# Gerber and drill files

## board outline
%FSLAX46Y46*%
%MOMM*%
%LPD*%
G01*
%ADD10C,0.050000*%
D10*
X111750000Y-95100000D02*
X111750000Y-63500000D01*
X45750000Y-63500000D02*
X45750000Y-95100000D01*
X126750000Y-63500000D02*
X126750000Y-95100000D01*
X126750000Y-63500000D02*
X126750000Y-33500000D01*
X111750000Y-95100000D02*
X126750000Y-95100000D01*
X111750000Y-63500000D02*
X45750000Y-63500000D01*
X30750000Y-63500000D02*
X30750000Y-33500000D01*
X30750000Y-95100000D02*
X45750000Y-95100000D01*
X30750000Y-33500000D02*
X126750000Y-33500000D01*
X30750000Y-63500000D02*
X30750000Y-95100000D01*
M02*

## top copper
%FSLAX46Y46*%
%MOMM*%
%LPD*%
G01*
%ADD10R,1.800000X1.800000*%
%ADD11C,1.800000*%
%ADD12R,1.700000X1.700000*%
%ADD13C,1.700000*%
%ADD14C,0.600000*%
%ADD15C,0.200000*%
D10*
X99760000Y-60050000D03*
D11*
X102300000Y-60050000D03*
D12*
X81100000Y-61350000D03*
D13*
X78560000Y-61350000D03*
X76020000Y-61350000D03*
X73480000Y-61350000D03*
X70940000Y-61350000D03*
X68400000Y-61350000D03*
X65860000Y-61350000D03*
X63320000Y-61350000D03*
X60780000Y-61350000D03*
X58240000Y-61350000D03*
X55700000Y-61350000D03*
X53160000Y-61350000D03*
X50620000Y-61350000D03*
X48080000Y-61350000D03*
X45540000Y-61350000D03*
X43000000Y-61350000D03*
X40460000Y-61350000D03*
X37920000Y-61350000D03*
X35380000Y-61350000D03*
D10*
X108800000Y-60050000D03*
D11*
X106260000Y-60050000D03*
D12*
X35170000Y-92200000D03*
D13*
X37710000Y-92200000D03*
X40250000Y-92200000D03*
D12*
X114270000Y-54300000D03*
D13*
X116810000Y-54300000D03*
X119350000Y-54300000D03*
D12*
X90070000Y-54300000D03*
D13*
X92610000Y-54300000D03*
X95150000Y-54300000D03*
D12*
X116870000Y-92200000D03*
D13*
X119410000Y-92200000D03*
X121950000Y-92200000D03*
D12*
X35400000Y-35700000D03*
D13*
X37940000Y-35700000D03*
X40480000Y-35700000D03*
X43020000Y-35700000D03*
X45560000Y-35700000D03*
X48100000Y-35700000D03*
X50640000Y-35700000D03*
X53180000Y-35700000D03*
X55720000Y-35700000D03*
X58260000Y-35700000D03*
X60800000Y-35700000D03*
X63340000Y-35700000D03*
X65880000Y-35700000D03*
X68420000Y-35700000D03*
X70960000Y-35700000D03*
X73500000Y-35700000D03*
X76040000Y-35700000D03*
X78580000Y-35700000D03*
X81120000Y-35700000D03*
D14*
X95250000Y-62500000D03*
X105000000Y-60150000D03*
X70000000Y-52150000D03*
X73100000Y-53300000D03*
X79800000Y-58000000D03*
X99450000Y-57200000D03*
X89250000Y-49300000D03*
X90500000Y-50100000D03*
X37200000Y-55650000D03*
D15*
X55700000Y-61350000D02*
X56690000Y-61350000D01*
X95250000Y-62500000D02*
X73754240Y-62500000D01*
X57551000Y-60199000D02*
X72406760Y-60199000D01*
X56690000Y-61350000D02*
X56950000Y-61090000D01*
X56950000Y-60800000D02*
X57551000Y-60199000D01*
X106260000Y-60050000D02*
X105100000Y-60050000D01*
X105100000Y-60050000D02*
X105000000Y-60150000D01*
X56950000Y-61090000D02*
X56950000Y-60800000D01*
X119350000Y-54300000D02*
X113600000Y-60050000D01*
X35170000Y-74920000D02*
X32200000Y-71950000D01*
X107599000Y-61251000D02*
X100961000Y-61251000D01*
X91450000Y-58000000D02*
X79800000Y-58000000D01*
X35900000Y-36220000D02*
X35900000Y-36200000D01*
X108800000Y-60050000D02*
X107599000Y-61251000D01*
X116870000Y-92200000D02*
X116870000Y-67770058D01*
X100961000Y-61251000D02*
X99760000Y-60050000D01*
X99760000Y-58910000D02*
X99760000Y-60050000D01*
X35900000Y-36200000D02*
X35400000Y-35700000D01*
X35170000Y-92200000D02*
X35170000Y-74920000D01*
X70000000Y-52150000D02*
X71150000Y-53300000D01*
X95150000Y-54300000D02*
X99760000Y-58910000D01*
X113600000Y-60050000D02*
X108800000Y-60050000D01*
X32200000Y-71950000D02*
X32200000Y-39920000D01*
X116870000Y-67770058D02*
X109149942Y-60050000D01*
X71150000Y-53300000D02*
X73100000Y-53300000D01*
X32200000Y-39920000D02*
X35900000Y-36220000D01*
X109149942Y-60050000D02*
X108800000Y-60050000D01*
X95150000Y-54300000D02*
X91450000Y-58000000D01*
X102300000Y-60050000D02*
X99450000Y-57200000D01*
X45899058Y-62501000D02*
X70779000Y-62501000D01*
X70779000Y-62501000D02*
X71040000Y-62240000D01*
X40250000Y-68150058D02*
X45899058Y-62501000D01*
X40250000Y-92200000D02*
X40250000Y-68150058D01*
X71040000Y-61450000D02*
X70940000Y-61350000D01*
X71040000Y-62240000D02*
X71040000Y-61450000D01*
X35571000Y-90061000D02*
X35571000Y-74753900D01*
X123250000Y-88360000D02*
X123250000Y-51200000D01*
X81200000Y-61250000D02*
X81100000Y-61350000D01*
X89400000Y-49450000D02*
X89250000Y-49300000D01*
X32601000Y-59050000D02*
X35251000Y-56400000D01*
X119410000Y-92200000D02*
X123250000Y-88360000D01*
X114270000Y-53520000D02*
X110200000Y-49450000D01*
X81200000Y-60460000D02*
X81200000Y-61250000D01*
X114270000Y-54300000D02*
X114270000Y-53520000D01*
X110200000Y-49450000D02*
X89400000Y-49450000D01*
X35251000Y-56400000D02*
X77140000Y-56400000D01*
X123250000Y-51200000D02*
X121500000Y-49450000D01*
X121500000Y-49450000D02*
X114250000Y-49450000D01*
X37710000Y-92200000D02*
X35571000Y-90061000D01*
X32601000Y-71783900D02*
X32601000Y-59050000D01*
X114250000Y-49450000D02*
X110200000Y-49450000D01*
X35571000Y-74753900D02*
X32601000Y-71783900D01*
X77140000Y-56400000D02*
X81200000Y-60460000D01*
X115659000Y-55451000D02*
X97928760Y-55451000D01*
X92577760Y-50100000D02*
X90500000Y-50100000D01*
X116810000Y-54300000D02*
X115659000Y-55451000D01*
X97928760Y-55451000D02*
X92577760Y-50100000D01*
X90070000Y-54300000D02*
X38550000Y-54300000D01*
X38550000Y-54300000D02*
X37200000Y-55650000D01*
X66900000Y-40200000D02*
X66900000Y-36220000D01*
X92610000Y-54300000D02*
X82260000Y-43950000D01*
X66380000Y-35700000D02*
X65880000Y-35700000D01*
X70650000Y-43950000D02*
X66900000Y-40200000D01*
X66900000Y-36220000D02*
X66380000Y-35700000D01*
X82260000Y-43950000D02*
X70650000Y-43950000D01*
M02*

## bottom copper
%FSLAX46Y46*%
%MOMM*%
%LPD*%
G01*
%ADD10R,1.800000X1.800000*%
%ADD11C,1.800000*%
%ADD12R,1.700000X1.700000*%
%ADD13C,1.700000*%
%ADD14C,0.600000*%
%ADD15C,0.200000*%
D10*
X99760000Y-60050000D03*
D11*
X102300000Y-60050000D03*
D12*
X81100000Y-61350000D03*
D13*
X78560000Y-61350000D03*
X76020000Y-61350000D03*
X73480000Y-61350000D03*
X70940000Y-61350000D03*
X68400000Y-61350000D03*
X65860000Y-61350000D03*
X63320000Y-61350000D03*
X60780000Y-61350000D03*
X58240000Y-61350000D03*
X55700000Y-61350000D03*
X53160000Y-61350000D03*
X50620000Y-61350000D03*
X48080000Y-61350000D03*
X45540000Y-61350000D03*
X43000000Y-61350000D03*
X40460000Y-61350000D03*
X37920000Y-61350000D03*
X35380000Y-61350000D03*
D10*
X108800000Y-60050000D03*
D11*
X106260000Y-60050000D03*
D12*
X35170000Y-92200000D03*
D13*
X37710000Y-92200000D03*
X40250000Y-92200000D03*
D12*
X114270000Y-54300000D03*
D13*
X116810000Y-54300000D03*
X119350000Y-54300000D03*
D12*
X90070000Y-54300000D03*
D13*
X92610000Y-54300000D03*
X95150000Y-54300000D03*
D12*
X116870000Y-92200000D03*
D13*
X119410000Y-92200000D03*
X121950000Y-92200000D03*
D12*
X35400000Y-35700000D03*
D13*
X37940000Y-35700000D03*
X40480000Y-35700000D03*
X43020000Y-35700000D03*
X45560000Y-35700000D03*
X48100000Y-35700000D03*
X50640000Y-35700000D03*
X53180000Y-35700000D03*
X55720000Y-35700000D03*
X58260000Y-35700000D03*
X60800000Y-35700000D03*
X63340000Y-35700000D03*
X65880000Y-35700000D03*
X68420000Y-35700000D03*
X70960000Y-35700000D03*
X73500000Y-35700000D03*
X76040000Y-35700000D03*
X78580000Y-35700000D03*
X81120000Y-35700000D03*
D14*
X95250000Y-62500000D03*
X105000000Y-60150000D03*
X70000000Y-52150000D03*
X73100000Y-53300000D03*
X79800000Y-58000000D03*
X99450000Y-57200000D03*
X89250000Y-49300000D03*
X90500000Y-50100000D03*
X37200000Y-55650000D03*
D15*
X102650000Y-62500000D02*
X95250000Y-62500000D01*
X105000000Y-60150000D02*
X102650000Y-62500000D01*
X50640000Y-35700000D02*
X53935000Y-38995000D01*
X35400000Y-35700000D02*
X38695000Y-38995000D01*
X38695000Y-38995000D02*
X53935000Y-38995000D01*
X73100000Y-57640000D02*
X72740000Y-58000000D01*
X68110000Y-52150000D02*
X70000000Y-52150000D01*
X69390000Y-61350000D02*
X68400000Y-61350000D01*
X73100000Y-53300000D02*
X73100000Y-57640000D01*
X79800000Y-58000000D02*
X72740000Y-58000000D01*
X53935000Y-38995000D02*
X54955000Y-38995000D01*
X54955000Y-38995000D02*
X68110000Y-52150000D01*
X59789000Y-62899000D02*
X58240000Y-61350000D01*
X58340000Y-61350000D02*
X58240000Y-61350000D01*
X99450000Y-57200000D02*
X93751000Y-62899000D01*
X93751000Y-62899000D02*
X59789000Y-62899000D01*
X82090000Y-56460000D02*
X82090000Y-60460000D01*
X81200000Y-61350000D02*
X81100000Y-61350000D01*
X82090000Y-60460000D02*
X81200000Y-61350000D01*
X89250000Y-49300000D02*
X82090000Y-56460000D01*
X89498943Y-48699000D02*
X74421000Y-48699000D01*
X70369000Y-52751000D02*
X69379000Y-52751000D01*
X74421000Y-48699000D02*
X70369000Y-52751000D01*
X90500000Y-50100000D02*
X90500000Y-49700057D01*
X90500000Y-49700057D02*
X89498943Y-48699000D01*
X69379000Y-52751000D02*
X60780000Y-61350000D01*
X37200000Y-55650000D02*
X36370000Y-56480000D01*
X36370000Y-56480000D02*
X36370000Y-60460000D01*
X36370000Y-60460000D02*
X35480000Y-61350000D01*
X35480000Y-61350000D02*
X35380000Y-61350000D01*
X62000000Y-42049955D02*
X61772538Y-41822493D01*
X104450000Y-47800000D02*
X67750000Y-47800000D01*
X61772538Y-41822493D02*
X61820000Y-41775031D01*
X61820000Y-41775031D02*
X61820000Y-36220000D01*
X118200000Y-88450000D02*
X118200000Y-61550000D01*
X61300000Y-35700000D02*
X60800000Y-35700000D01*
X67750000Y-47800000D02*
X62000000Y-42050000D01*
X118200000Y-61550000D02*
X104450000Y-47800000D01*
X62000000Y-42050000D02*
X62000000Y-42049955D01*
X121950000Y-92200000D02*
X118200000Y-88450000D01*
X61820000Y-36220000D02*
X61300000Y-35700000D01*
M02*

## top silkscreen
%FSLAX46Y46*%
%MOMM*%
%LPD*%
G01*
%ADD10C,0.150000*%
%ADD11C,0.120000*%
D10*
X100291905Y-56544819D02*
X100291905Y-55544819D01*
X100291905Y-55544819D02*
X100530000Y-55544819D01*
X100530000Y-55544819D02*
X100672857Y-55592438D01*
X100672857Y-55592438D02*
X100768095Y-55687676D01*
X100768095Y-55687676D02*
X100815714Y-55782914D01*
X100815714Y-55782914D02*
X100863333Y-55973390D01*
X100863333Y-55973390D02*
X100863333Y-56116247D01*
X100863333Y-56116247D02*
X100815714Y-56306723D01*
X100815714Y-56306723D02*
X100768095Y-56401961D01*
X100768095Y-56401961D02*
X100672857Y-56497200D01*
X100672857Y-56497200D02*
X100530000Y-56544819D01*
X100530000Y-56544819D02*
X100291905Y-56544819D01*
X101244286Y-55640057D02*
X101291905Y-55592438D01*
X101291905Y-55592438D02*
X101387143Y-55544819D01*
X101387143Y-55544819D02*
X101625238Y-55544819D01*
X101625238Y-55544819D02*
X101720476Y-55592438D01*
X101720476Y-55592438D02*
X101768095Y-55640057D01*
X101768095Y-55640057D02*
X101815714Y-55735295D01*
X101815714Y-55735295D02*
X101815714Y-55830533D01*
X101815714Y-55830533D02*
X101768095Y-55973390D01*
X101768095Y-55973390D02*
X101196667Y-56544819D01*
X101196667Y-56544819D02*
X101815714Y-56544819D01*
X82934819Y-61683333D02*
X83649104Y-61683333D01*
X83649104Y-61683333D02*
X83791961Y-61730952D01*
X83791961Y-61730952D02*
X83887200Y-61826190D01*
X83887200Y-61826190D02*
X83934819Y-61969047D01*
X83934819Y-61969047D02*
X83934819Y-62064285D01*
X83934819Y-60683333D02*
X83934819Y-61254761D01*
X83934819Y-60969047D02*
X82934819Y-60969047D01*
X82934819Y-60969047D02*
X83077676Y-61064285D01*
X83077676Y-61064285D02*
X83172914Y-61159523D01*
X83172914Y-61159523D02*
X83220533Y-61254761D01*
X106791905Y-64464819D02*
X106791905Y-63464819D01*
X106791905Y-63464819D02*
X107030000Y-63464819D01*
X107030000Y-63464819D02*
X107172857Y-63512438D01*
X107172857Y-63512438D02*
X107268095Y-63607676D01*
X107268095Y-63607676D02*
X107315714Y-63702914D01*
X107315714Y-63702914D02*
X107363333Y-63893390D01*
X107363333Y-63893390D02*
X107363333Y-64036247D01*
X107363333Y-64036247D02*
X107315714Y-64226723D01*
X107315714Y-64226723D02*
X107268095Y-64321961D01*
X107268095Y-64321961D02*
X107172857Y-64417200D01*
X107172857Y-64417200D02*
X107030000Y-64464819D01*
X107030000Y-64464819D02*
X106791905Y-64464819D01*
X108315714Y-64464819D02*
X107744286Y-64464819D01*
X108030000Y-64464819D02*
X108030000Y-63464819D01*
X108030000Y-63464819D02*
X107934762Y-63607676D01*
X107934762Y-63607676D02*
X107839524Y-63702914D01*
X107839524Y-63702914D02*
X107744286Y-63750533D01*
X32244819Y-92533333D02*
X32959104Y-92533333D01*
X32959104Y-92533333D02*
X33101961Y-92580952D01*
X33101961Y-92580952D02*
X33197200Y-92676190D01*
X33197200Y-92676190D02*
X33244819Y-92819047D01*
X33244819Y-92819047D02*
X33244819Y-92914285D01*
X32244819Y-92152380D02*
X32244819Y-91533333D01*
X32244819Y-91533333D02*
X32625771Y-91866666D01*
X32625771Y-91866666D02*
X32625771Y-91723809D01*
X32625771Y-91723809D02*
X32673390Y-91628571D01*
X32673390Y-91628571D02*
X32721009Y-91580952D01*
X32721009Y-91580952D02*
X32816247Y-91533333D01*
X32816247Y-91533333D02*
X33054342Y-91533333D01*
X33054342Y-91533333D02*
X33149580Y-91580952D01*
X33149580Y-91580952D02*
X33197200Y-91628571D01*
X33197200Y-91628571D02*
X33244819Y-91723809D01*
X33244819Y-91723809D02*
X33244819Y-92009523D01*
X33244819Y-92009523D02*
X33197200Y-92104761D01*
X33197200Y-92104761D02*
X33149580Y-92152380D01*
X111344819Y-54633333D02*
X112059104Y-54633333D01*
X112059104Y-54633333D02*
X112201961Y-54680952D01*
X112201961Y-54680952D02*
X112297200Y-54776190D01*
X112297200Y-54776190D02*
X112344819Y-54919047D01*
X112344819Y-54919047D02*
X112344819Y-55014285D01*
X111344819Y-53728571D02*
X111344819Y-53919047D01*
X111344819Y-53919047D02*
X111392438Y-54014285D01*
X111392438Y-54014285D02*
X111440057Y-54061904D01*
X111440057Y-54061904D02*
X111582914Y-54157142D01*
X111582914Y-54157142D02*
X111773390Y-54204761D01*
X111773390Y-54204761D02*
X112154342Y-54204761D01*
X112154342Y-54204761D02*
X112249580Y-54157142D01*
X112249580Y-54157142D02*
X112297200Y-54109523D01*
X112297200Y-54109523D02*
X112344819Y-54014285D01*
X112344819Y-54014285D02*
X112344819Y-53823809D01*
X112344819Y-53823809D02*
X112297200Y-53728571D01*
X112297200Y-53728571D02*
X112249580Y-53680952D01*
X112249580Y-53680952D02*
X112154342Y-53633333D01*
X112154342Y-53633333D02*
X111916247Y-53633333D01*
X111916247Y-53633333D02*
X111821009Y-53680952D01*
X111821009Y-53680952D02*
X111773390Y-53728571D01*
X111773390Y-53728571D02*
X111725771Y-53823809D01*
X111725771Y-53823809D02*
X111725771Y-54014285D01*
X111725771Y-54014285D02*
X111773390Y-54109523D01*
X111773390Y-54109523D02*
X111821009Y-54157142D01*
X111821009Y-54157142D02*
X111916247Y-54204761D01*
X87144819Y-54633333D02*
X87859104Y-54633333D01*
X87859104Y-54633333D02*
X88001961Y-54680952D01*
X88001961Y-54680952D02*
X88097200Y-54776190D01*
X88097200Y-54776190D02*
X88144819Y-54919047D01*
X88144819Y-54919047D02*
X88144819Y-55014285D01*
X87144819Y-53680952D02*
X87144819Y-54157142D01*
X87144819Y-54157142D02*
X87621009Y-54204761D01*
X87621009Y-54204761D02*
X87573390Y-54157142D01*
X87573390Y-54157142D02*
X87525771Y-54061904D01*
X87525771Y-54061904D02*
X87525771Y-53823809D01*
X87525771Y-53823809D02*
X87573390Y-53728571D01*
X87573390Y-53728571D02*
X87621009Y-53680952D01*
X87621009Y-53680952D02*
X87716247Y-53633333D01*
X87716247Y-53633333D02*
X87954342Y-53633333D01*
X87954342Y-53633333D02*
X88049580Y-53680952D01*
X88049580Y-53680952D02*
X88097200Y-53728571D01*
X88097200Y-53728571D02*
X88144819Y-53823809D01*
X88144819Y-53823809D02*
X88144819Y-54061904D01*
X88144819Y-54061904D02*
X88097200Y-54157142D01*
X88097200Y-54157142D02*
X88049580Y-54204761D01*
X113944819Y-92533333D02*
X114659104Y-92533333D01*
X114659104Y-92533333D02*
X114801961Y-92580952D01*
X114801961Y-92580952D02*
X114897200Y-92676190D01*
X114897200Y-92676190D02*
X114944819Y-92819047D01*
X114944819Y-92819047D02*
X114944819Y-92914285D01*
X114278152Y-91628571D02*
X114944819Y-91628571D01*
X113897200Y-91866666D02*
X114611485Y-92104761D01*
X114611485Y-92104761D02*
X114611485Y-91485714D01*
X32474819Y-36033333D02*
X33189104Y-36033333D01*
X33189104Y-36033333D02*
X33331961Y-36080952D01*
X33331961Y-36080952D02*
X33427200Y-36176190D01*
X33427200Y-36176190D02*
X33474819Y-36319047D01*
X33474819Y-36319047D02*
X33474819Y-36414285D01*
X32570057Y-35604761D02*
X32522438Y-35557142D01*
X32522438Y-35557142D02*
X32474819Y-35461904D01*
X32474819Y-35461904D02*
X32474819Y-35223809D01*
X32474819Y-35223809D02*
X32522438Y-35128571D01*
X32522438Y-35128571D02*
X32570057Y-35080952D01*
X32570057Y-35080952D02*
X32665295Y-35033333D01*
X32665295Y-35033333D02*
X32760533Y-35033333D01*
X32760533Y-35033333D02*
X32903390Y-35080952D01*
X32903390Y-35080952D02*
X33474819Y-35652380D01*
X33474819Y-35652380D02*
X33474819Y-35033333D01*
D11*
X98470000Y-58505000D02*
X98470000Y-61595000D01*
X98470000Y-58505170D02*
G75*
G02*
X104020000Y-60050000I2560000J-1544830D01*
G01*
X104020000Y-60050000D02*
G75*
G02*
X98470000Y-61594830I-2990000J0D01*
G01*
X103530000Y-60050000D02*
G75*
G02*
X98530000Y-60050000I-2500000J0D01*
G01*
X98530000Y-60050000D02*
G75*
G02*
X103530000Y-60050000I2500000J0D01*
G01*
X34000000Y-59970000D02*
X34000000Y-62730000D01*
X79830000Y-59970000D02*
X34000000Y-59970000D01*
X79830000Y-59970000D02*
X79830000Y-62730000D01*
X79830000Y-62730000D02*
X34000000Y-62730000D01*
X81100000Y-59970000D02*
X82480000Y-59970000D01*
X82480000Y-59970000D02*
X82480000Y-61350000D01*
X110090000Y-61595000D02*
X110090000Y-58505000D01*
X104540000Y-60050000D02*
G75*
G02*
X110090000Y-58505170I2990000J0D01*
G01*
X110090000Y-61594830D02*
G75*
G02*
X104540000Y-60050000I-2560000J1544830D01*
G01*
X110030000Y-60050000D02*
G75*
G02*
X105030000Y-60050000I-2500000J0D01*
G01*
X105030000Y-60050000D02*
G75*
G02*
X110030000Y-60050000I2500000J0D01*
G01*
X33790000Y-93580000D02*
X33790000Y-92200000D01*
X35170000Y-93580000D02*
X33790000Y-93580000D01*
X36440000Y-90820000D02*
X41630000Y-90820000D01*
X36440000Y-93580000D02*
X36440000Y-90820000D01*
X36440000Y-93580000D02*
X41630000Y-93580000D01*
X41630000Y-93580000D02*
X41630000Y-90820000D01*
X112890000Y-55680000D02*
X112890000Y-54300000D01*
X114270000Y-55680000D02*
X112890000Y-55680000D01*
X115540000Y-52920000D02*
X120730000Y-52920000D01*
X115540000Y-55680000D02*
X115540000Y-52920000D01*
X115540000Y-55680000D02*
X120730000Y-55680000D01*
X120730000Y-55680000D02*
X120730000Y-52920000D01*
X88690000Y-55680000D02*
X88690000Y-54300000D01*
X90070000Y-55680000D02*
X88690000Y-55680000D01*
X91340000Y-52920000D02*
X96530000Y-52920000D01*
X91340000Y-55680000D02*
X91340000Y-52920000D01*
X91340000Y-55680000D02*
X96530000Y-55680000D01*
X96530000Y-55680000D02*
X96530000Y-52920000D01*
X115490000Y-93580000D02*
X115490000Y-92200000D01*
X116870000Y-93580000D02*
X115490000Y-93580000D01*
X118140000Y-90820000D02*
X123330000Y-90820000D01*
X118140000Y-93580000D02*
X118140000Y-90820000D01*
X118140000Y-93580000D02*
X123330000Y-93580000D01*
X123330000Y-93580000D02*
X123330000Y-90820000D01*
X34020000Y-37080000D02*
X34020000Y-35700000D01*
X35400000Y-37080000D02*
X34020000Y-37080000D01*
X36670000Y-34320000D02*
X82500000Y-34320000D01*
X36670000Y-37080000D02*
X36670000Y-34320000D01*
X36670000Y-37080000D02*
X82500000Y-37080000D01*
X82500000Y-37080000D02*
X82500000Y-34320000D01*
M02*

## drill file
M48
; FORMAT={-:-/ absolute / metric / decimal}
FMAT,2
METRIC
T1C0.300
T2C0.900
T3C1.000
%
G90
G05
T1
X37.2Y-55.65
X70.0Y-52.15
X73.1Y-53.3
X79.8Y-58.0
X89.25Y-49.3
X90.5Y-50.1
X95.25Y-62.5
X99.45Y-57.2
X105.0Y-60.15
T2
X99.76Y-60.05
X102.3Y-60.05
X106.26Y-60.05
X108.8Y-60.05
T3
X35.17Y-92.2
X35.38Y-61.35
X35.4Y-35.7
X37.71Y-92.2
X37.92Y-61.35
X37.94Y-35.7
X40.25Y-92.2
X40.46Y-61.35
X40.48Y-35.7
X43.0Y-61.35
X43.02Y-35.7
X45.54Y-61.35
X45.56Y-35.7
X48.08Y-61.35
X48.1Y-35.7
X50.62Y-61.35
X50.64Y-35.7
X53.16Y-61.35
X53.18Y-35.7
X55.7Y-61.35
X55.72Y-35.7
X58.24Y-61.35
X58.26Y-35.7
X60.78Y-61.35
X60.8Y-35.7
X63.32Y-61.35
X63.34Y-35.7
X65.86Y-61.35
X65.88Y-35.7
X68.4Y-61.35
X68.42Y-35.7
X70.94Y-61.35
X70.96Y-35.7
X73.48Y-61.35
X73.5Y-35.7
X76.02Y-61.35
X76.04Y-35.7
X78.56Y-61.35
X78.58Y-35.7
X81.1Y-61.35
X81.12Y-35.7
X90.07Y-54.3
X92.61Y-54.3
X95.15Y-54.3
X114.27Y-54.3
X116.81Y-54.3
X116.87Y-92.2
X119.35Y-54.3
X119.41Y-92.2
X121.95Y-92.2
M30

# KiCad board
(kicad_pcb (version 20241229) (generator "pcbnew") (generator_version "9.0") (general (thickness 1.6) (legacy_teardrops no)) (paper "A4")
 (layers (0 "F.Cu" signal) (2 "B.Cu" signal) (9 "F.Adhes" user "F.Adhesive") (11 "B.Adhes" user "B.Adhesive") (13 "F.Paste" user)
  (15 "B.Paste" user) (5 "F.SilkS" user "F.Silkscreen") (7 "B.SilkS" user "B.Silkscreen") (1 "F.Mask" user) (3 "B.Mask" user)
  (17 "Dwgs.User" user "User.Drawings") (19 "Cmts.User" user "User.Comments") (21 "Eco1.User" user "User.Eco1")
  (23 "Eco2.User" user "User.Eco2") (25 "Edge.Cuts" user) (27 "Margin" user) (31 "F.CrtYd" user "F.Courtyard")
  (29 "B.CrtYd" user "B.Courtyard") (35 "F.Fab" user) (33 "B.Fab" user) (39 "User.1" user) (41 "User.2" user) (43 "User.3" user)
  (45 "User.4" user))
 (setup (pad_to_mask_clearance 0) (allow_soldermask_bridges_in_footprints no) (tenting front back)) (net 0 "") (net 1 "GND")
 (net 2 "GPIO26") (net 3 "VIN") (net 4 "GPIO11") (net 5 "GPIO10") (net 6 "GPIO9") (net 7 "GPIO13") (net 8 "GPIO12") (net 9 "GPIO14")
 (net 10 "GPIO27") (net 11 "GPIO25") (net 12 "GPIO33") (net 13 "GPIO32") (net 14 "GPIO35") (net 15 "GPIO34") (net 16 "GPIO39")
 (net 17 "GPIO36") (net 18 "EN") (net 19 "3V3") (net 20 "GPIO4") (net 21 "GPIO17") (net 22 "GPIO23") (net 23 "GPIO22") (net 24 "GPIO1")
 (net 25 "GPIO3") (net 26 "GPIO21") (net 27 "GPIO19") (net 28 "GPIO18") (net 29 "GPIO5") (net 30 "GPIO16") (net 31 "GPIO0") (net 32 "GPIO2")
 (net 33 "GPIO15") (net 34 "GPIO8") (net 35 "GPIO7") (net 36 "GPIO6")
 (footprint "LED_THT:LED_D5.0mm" (layer "F.Cu") (at 99.76 60.05)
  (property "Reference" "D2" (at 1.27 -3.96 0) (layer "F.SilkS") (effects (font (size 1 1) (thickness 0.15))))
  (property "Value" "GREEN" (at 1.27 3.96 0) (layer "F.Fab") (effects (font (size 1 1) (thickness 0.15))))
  (fp_line (start -1.29 -1.545) (end -1.29 1.545) (stroke (width 0.12) (type solid)) (layer "F.SilkS"))
  (fp_arc (start -1.29 -1.54483) (mid 2.071779 -2.880495) (end 4.26 0) (stroke (width 0.12) (type solid)) (layer "F.SilkS"))
  (fp_arc (start 4.26 0) (mid 2.071779 2.880495) (end -1.29 1.54483) (stroke (width 0.12) (type solid)) (layer "F.SilkS"))
  (fp_circle (center 1.27 0) (end 3.77 0) (stroke (width 0.12) (type solid)) (fill no) (layer "F.SilkS"))
  (pad "1" thru_hole rect (at 0 0) (size 1.8 1.8) (drill 0.9) (layers "*.Cu" "*.Mask") (remove_unused_layers no) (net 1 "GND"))
  (pad "2" thru_hole circle (at 2.54 0) (size 1.8 1.8) (drill 0.9) (layers "*.Cu" "*.Mask") (remove_unused_layers no) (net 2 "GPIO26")))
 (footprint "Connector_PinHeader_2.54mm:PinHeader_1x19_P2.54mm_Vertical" (layer "F.Cu") (at 81.1 61.35 -90)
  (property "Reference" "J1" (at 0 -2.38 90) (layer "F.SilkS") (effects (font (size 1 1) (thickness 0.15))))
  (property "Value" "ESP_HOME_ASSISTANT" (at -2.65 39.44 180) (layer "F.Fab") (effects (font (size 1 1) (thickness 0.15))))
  (fp_line (start -1.38 47.1) (end 1.38 47.1) (stroke (width 0.12) (type solid)) (layer "F.SilkS"))
  (fp_line (start -1.38 1.27) (end -1.38 47.1) (stroke (width 0.12) (type solid)) (layer "F.SilkS"))
  (fp_line (start -1.38 1.27) (end 1.38 1.27) (stroke (width 0.12) (type solid)) (layer "F.SilkS"))
  (fp_line (start 1.38 1.27) (end 1.38 47.1) (stroke (width 0.12) (type solid)) (layer "F.SilkS"))
  (fp_line (start -1.38 0) (end -1.38 -1.38) (stroke (width 0.12) (type solid)) (layer "F.SilkS"))
  (fp_line (start -1.38 -1.38) (end 0 -1.38) (stroke (width 0.12) (type solid)) (layer "F.SilkS"))
  (pad "1" thru_hole rect (at 0 0 270) (size 1.7 1.7) (drill 1) (layers "*.Cu" "*.Mask") (remove_unused_layers no) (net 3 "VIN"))
  (pad "2" thru_hole circle (at 0 2.54 270) (size 1.7 1.7) (drill 1) (layers "*.Cu" "*.Mask") (remove_unused_layers no) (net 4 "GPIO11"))
  (pad "3" thru_hole circle (at 0 5.08 270) (size 1.7 1.7) (drill 1) (layers "*.Cu" "*.Mask") (remove_unused_layers no) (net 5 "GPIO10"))
  (pad "4" thru_hole circle (at 0 7.62 270) (size 1.7 1.7) (drill 1) (layers "*.Cu" "*.Mask") (remove_unused_layers no) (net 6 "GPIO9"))
  (pad "5" thru_hole circle (at 0 10.16 270) (size 1.7 1.7) (drill 1) (layers "*.Cu" "*.Mask") (remove_unused_layers no) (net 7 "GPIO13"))
  (pad "6" thru_hole circle (at 0 12.7 270) (size 1.7 1.7) (drill 1) (layers "*.Cu" "*.Mask") (remove_unused_layers no) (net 1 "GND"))
  (pad "7" thru_hole circle (at 0 15.24 270) (size 1.7 1.7) (drill 1) (layers "*.Cu" "*.Mask") (remove_unused_layers no) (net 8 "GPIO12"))
  (pad "8" thru_hole circle (at 0 17.78 270) (size 1.7 1.7) (drill 1) (layers "*.Cu" "*.Mask") (remove_unused_layers no) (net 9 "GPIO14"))
  (pad "9" thru_hole circle (at 0 20.32 270) (size 1.7 1.7) (drill 1) (layers "*.Cu" "*.Mask") (remove_unused_layers no) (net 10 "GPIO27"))
  (pad "10" thru_hole circle (at 0 22.86 270) (size 1.7 1.7) (drill 1) (layers "*.Cu" "*.Mask") (remove_unused_layers no) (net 2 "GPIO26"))
  (pad "11" thru_hole circle (at 0 25.4 270) (size 1.7 1.7) (drill 1) (layers "*.Cu" "*.Mask") (remove_unused_layers no) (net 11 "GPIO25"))
  (pad "12" thru_hole circle (at 0 27.94 270) (size 1.7 1.7) (drill 1) (layers "*.Cu" "*.Mask") (remove_unused_layers no) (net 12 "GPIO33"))
  (pad "13" thru_hole circle (at 0 30.48 270) (size 1.7 1.7) (drill 1) (layers "*.Cu" "*.Mask") (remove_unused_layers no) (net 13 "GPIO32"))
  (pad "14" thru_hole circle (at 0 33.02 270) (size 1.7 1.7) (drill 1) (layers "*.Cu" "*.Mask") (remove_unused_layers no) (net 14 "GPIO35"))
  (pad "15" thru_hole circle (at 0 35.56 270) (size 1.7 1.7) (drill 1) (layers "*.Cu" "*.Mask") (remove_unused_layers no) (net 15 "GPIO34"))
  (pad "16" thru_hole circle (at 0 38.1 270) (size 1.7 1.7) (drill 1) (layers "*.Cu" "*.Mask") (remove_unused_layers no) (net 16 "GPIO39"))
  (pad "17" thru_hole circle (at 0 40.64 270) (size 1.7 1.7) (drill 1) (layers "*.Cu" "*.Mask") (remove_unused_layers no) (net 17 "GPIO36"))
  (pad "18" thru_hole circle (at 0 43.18 270) (size 1.7 1.7) (drill 1) (layers "*.Cu" "*.Mask") (remove_unused_layers no) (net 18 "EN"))
  (pad "19" thru_hole circle (at 0 45.72 270) (size 1.7 1.7) (drill 1) (layers "*.Cu" "*.Mask") (remove_unused_layers no) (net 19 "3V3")))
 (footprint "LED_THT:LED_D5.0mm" (layer "F.Cu") (at 108.8 60.05 180)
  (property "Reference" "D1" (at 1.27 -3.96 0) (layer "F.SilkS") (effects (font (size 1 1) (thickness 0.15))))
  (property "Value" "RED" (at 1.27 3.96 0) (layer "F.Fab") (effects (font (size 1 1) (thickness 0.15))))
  (fp_line (start -1.29 -1.545) (end -1.29 1.545) (stroke (width 0.12) (type solid)) (layer "F.SilkS"))
  (fp_arc (start 4.26 0) (mid 2.071779 2.880495) (end -1.29 1.54483) (stroke (width 0.12) (type solid)) (layer "F.SilkS"))
  (fp_arc (start -1.29 -1.54483) (mid 2.071779 -2.880495) (end 4.26 0) (stroke (width 0.12) (type solid)) (layer "F.SilkS"))
  (fp_circle (center 1.27 0) (end 3.77 0) (stroke (width 0.12) (type solid)) (fill no) (layer "F.SilkS"))
  (pad "1" thru_hole rect (at 0 0 180) (size 1.8 1.8) (drill 0.9) (layers "*.Cu" "*.Mask") (remove_unused_layers no) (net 1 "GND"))
  (pad "2" thru_hole circle (at 2.54 0 180) (size 1.8 1.8) (drill 0.9) (layers "*.Cu" "*.Mask") (remove_unused_layers no) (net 11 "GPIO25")))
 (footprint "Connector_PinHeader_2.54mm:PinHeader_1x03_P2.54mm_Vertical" (layer "F.Cu") (at 35.17 92.2 90)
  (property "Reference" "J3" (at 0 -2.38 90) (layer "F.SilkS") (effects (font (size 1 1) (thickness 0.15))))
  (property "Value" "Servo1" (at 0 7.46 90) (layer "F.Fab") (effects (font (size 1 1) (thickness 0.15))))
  (fp_line (start -1.38 -1.38) (end 0 -1.38) (stroke (width 0.12) (type solid)) (layer "F.SilkS"))
  (fp_line (start -1.38 0) (end -1.38 -1.38) (stroke (width 0.12) (type solid)) (layer "F.SilkS"))
  (fp_line (start 1.38 1.27) (end 1.38 6.46) (stroke (width 0.12) (type solid)) (layer "F.SilkS"))
  (fp_line (start -1.38 1.27) (end 1.38 1.27) (stroke (width 0.12) (type solid)) (layer "F.SilkS"))
  (fp_line (start -1.38 1.27) (end -1.38 6.46) (stroke (width 0.12) (type solid)) (layer "F.SilkS"))
  (fp_line (start -1.38 6.46) (end 1.38 6.46) (stroke (width 0.12) (type solid)) (layer "F.SilkS"))
  (pad "1" thru_hole rect (at 0 0 90) (size 1.7 1.7) (drill 1) (layers "*.Cu" "*.Mask") (remove_unused_layers no) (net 1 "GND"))
  (pad "2" thru_hole circle (at 0 2.54 90) (size 1.7 1.7) (drill 1) (layers "*.Cu" "*.Mask") (remove_unused_layers no) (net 3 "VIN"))
  (pad "3" thru_hole circle (at 0 5.08 90) (size 1.7 1.7) (drill 1) (layers "*.Cu" "*.Mask") (remove_unused_layers no) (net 7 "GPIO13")))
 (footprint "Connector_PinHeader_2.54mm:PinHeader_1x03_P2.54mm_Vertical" (layer "F.Cu") (at 114.27 54.3 90)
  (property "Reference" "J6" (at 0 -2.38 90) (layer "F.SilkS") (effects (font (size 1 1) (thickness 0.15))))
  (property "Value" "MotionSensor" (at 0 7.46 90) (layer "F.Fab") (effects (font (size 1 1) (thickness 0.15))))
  (fp_line (start -1.38 -1.38) (end 0 -1.38) (stroke (width 0.12) (type solid)) (layer "F.SilkS"))
  (fp_line (start -1.38 0) (end -1.38 -1.38) (stroke (width 0.12) (type solid)) (layer "F.SilkS"))
  (fp_line (start 1.38 1.27) (end 1.38 6.46) (stroke (width 0.12) (type solid)) (layer "F.SilkS"))
  (fp_line (start -1.38 1.27) (end 1.38 1.27) (stroke (width 0.12) (type solid)) (layer "F.SilkS"))
  (fp_line (start -1.38 1.27) (end -1.38 6.46) (stroke (width 0.12) (type solid)) (layer "F.SilkS"))
  (fp_line (start -1.38 6.46) (end 1.38 6.46) (stroke (width 0.12) (type solid)) (layer "F.SilkS"))
  (pad "1" thru_hole rect (at 0 0 90) (size 1.7 1.7) (drill 1) (layers "*.Cu" "*.Mask") (remove_unused_layers no) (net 3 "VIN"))
  (pad "2" thru_hole circle (at 0 2.54 90) (size 1.7 1.7) (drill 1) (layers "*.Cu" "*.Mask") (remove_unused_layers no) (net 10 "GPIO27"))
  (pad "3" thru_hole circle (at 0 5.08 90) (size 1.7 1.7) (drill 1) (layers "*.Cu" "*.Mask") (remove_unused_layers no) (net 1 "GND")))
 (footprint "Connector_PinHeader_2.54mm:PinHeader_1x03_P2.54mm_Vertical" (layer "F.Cu") (at 90.07 54.3 90)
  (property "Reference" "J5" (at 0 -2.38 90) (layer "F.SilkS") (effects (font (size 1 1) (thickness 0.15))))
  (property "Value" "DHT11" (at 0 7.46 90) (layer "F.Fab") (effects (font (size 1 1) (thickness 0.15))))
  (fp_line (start -1.38 -1.38) (end 0 -1.38) (stroke (width 0.12) (type solid)) (layer "F.SilkS"))
  (fp_line (start -1.38 0) (end -1.38 -1.38) (stroke (width 0.12) (type solid)) (layer "F.SilkS"))
  (fp_line (start 1.38 1.27) (end 1.38 6.46) (stroke (width 0.12) (type solid)) (layer "F.SilkS"))
  (fp_line (start -1.38 1.27) (end 1.38 1.27) (stroke (width 0.12) (type solid)) (layer "F.SilkS"))
  (fp_line (start -1.38 1.27) (end -1.38 6.46) (stroke (width 0.12) (type solid)) (layer "F.SilkS"))
  (fp_line (start -1.38 6.46) (end 1.38 6.46) (stroke (width 0.12) (type solid)) (layer "F.SilkS"))
  (pad "1" thru_hole rect (at 0 0 90) (size 1.7 1.7) (drill 1) (layers "*.Cu" "*.Mask") (remove_unused_layers no) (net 19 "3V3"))
  (pad "2" thru_hole circle (at 0 2.54 90) (size 1.7 1.7) (drill 1) (layers "*.Cu" "*.Mask") (remove_unused_layers no) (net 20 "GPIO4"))
  (pad "3" thru_hole circle (at 0 5.08 90) (size 1.7 1.7) (drill 1) (layers "*.Cu" "*.Mask") (remove_unused_layers no) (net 1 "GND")))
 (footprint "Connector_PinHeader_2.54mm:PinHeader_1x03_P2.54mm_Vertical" (layer "F.Cu") (at 116.87 92.2 90)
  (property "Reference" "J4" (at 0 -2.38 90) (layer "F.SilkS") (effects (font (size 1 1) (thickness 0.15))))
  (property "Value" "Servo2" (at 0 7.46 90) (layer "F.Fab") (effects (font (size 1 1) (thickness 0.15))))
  (fp_line (start -1.38 -1.38) (end 0 -1.38) (stroke (width 0.12) (type solid)) (layer "F.SilkS"))
  (fp_line (start -1.38 0) (end -1.38 -1.38) (stroke (width 0.12) (type solid)) (layer "F.SilkS"))
  (fp_line (start 1.38 1.27) (end 1.38 6.46) (stroke (width 0.12) (type solid)) (layer "F.SilkS"))
  (fp_line (start -1.38 1.27) (end 1.38 1.27) (stroke (width 0.12) (type solid)) (layer "F.SilkS"))
  (fp_line (start -1.38 1.27) (end -1.38 6.46) (stroke (width 0.12) (type solid)) (layer "F.SilkS"))
  (fp_line (start -1.38 6.46) (end 1.38 6.46) (stroke (width 0.12) (type solid)) (layer "F.SilkS"))
  (pad "1" thru_hole rect (at 0 0 90) (size 1.7 1.7) (drill 1) (layers "*.Cu" "*.Mask") (remove_unused_layers no) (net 1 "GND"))
  (pad "2" thru_hole circle (at 0 2.54 90) (size 1.7 1.7) (drill 1) (layers "*.Cu" "*.Mask") (remove_unused_layers no) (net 3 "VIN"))
  (pad "3" thru_hole circle (at 0 5.08 90) (size 1.7 1.7) (drill 1) (layers "*.Cu" "*.Mask") (remove_unused_layers no) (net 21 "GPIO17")))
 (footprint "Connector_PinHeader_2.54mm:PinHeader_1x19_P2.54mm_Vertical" (layer "F.Cu") (at 35.4 35.7 90)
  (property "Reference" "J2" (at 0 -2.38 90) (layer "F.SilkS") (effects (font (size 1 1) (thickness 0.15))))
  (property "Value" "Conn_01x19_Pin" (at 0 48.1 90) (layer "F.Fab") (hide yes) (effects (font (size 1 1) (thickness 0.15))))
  (fp_line (start -1.38 -1.38) (end 0 -1.38) (stroke (width 0.12) (type solid)) (layer "F.SilkS"))
  (fp_line (start -1.38 0) (end -1.38 -1.38) (stroke (width 0.12) (type solid)) (layer "F.SilkS"))
  (fp_line (start 1.38 1.27) (end 1.38 47.1) (stroke (width 0.12) (type solid)) (layer "F.SilkS"))
  (fp_line (start -1.38 1.27) (end 1.38 1.27) (stroke (width 0.12) (type solid)) (layer "F.SilkS"))
  (fp_line (start -1.38 1.27) (end -1.38 47.1) (stroke (width 0.12) (type solid)) (layer "F.SilkS"))
  (fp_line (start -1.38 47.1) (end 1.38 47.1) (stroke (width 0.12) (type solid)) (layer "F.SilkS"))
  (pad "1" thru_hole rect (at 0 0 90) (size 1.7 1.7) (drill 1) (layers "*.Cu" "*.Mask") (remove_unused_layers no) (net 1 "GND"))
  (pad "2" thru_hole circle (at 0 2.54 90) (size 1.7 1.7) (drill 1) (layers "*.Cu" "*.Mask") (remove_unused_layers no) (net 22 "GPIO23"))
  (pad "3" thru_hole circle (at 0 5.08 90) (size 1.7 1.7) (drill 1) (layers "*.Cu" "*.Mask") (remove_unused_layers no) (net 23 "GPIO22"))
  (pad "4" thru_hole circle (at 0 7.62 90) (size 1.7 1.7) (drill 1) (layers "*.Cu" "*.Mask") (remove_unused_layers no) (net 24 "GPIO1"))
  (pad "5" thru_hole circle (at 0 10.16 90) (size 1.7 1.7) (drill 1) (layers "*.Cu" "*.Mask") (remove_unused_layers no) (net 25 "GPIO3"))
  (pad "6" thru_hole circle (at 0 12.7 90) (size 1.7 1.7) (drill 1) (layers "*.Cu" "*.Mask") (remove_unused_layers no) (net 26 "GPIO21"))
  (pad "7" thru_hole circle (at 0 15.24 90) (size 1.7 1.7) (drill 1) (layers "*.Cu" "*.Mask") (remove_unused_layers no) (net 1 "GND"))
  (pad "8" thru_hole circle (at 0 17.78 90) (size 1.7 1.7) (drill 1) (layers "*.Cu" "*.Mask") (remove_unused_layers no) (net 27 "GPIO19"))
  (pad "9" thru_hole circle (at 0 20.32 90) (size 1.7 1.7) (drill 1) (layers "*.Cu" "*.Mask") (remove_unused_layers no) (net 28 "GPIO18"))
  (pad "10" thru_hole circle (at 0 22.86 90) (size 1.7 1.7) (drill 1) (layers "*.Cu" "*.Mask") (remove_unused_layers no) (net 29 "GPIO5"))
  (pad "11" thru_hole circle (at 0 25.4 90) (size 1.7 1.7) (drill 1) (layers "*.Cu" "*.Mask") (remove_unused_layers no) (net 21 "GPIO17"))
  (pad "12" thru_hole circle (at 0 27.94 90) (size 1.7 1.7) (drill 1) (layers "*.Cu" "*.Mask") (remove_unused_layers no) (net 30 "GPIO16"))
  (pad "13" thru_hole circle (at 0 30.48 90) (size 1.7 1.7) (drill 1) (layers "*.Cu" "*.Mask") (remove_unused_layers no) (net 20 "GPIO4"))
  (pad "14" thru_hole circle (at 0 33.02 90) (size 1.7 1.7) (drill 1) (layers "*.Cu" "*.Mask") (remove_unused_layers no) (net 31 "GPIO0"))
  (pad "15" thru_hole circle (at 0 35.56 90) (size 1.7 1.7) (drill 1) (layers "*.Cu" "*.Mask") (remove_unused_layers no) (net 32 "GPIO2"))
  (pad "16" thru_hole circle (at 0 38.1 90) (size 1.7 1.7) (drill 1) (layers "*.Cu" "*.Mask") (remove_unused_layers no) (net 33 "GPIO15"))
  (pad "17" thru_hole circle (at 0 40.64 90) (size 1.7 1.7) (drill 1) (layers "*.Cu" "*.Mask") (remove_unused_layers no) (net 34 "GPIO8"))
  (pad "18" thru_hole circle (at 0 43.18 90) (size 1.7 1.7) (drill 1) (layers "*.Cu" "*.Mask") (remove_unused_layers no) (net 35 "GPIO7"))
  (pad "19" thru_hole circle (at 0 45.72 90) (size 1.7 1.7) (drill 1) (layers "*.Cu" "*.Mask") (remove_unused_layers no) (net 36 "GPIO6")))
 (gr_line (start 111.75 95.1) (end 111.75 63.5) (stroke (width 0.05) (type default)) (layer "Edge.Cuts"))
 (gr_line (start 45.75 63.5) (end 45.75 95.1) (stroke (width 0.05) (type default)) (layer "Edge.Cuts"))
 (gr_line (start 126.75 63.5) (end 126.75 95.1) (stroke (width 0.05) (type default)) (layer "Edge.Cuts"))
 (gr_line (start 126.75 63.5) (end 126.75 33.5) (stroke (width 0.05) (type default)) (layer "Edge.Cuts"))
 (gr_line (start 111.75 95.1) (end 126.75 95.1) (stroke (width 0.05) (type default)) (layer "Edge.Cuts"))
 (gr_line (start 111.75 63.5) (end 45.75 63.5) (stroke (width 0.05) (type default)) (layer "Edge.Cuts"))
 (gr_line (start 30.75 63.5) (end 30.75 33.5) (stroke (width 0.05) (type default)) (layer "Edge.Cuts"))
 (gr_line (start 30.75 95.1) (end 45.75 95.1) (stroke (width 0.05) (type default)) (layer "Edge.Cuts"))
 (gr_line (start 30.75 33.5) (end 126.75 33.5) (stroke (width 0.05) (type default)) (layer "Edge.Cuts"))
 (gr_line (start 30.75 63.5) (end 30.75 95.1) (stroke (width 0.05) (type default)) (layer "Edge.Cuts"))
 (segment (start 55.7 61.35) (end 56.69 61.35) (width 0.2) (layer "F.Cu") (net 11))
 (segment (start 95.25 62.5) (end 73.75424 62.5) (width 0.2) (layer "F.Cu") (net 11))
 (segment (start 57.551 60.199) (end 72.40676 60.199) (width 0.2) (layer "F.Cu") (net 11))
 (segment (start 56.69 61.35) (end 56.95 61.09) (width 0.2) (layer "F.Cu") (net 11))
 (segment (start 56.95 60.8) (end 57.551 60.199) (width 0.2) (layer "F.Cu") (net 11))
 (segment (start 106.26 60.05) (end 105.1 60.05) (width 0.2) (layer "F.Cu") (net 11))
 (segment (start 105.1 60.05) (end 105 60.15) (width 0.2) (layer "F.Cu") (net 11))
 (segment (start 56.95 61.09) (end 56.95 60.8) (width 0.2) (layer "F.Cu") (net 11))
 (via (at 95.25 62.5) (size 0.6) (drill 0.3) (layers "F.Cu" "B.Cu") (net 11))
 (via (at 105 60.15) (size 0.6) (drill 0.3) (layers "F.Cu" "B.Cu") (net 11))
 (segment (start 102.65 62.5) (end 95.25 62.5) (width 0.2) (layer "B.Cu") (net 11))
 (segment (start 105 60.15) (end 102.65 62.5) (width 0.2) (layer "B.Cu") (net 11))
 (segment (start 119.35 54.3) (end 113.6 60.05) (width 0.2) (layer "F.Cu") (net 1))
 (segment (start 35.17 74.92) (end 32.2 71.95) (width 0.2) (layer "F.Cu") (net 1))
 (segment (start 107.599 61.251) (end 100.961 61.251) (width 0.2) (layer "F.Cu") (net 1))
 (segment (start 91.45 58) (end 79.8 58) (width 0.2) (layer "F.Cu") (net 1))
 (segment (start 35.9 36.22) (end 35.9 36.2) (width 0.2) (layer "F.Cu") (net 1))
 (segment (start 108.8 60.05) (end 107.599 61.251) (width 0.2) (layer "F.Cu") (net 1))
 (segment (start 116.87 92.2) (end 116.87 67.770058) (width 0.2) (layer "F.Cu") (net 1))
 (segment (start 100.961 61.251) (end 99.76 60.05) (width 0.2) (layer "F.Cu") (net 1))
 (segment (start 99.76 58.91) (end 99.76 60.05) (width 0.2) (layer "F.Cu") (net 1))
 (segment (start 35.9 36.2) (end 35.4 35.7) (width 0.2) (layer "F.Cu") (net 1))
 (segment (start 35.17 92.2) (end 35.17 74.92) (width 0.2) (layer "F.Cu") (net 1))
 (segment (start 70 52.15) (end 71.15 53.3) (width 0.2) (layer "F.Cu") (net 1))
 (segment (start 95.15 54.3) (end 99.76 58.91) (width 0.2) (layer "F.Cu") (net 1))
 (segment (start 113.6 60.05) (end 108.8 60.05) (width 0.2) (layer "F.Cu") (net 1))
 (segment (start 32.2 71.95) (end 32.2 39.92) (width 0.2) (layer "F.Cu") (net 1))
 (segment (start 116.87 67.770058) (end 109.149942 60.05) (width 0.2) (layer "F.Cu") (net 1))
 (segment (start 71.15 53.3) (end 73.1 53.3) (width 0.2) (layer "F.Cu") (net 1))
 (segment (start 32.2 39.92) (end 35.9 36.22) (width 0.2) (layer "F.Cu") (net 1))
 (segment (start 109.149942 60.05) (end 108.8 60.05) (width 0.2) (layer "F.Cu") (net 1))
 (segment (start 95.15 54.3) (end 91.45 58) (width 0.2) (layer "F.Cu") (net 1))
 (via (at 70 52.15) (size 0.6) (drill 0.3) (layers "F.Cu" "B.Cu") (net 1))
 (via (at 73.1 53.3) (size 0.6) (drill 0.3) (layers "F.Cu" "B.Cu") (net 1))
 (via (at 79.8 58) (size 0.6) (drill 0.3) (layers "F.Cu" "B.Cu") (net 1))
 (segment (start 50.64 35.7) (end 53.935 38.995) (width 0.2) (layer "B.Cu") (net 1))
 (segment (start 35.4 35.7) (end 38.695 38.995) (width 0.2) (layer "B.Cu") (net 1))
 (segment (start 38.695 38.995) (end 53.935 38.995) (width 0.2) (layer "B.Cu") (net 1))
 (segment (start 73.1 57.64) (end 72.74 58) (width 0.2) (layer "B.Cu") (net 1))
 (segment (start 68.11 52.15) (end 70 52.15) (width 0.2) (layer "B.Cu") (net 1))
 (segment (start 69.39 61.35) (end 68.4 61.35) (width 0.2) (layer "B.Cu") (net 1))
 (segment (start 73.1 53.3) (end 73.1 57.64) (width 0.2) (layer "B.Cu") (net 1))
 (segment (start 79.8 58) (end 72.74 58) (width 0.2) (layer "B.Cu") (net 1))
 (segment (start 53.935 38.995) (end 54.955 38.995) (width 0.2) (layer "B.Cu") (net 1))
 (segment (start 54.955 38.995) (end 68.11 52.15) (width 0.2) (layer "B.Cu") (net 1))
 (segment (start 102.3 60.05) (end 99.45 57.2) (width 0.2) (layer "F.Cu") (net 2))
 (via (at 99.45 57.2) (size 0.6) (drill 0.3) (layers "F.Cu" "B.Cu") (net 2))
 (segment (start 59.789 62.899) (end 58.24 61.35) (width 0.2) (layer "B.Cu") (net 2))
 (segment (start 58.34 61.35) (end 58.24 61.35) (width 0.2) (layer "B.Cu") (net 2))
 (segment (start 99.45 57.2) (end 93.751 62.899) (width 0.2) (layer "B.Cu") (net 2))
 (segment (start 93.751 62.899) (end 59.789 62.899) (width 0.2) (layer "B.Cu") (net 2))
 (segment (start 45.899058 62.501) (end 70.779 62.501) (width 0.2) (layer "F.Cu") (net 7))
 (segment (start 70.779 62.501) (end 71.04 62.24) (width 0.2) (layer "F.Cu") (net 7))
 (segment (start 40.25 68.150058) (end 45.899058 62.501) (width 0.2) (layer "F.Cu") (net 7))
 (segment (start 40.25 92.2) (end 40.25 68.150058) (width 0.2) (layer "F.Cu") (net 7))
 (segment (start 71.04 61.45) (end 70.94 61.35) (width 0.2) (layer "F.Cu") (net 7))
 (segment (start 71.04 62.24) (end 71.04 61.45) (width 0.2) (layer "F.Cu") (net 7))
 (segment (start 35.571 90.061) (end 35.571 74.7539) (width 0.2) (layer "F.Cu") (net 3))
 (segment (start 123.25 88.36) (end 123.25 51.2) (width 0.2) (layer "F.Cu") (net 3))
 (segment (start 81.2 61.25) (end 81.1 61.35) (width 0.2) (layer "F.Cu") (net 3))
 (segment (start 89.4 49.45) (end 89.25 49.3) (width 0.2) (layer "F.Cu") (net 3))
 (segment (start 32.601 59.05) (end 35.251 56.4) (width 0.2) (layer "F.Cu") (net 3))
 (segment (start 119.41 92.2) (end 123.25 88.36) (width 0.2) (layer "F.Cu") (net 3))
 (segment (start 114.27 53.52) (end 110.2 49.45) (width 0.2) (layer "F.Cu") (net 3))
 (segment (start 81.2 60.46) (end 81.2 61.25) (width 0.2) (layer "F.Cu") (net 3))
 (segment (start 114.27 54.3) (end 114.27 53.52) (width 0.2) (layer "F.Cu") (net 3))
 (segment (start 110.2 49.45) (end 89.4 49.45) (width 0.2) (layer "F.Cu") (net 3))
 (segment (start 35.251 56.4) (end 77.14 56.4) (width 0.2) (layer "F.Cu") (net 3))
 (segment (start 123.25 51.2) (end 121.5 49.45) (width 0.2) (layer "F.Cu") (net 3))
 (segment (start 121.5 49.45) (end 114.25 49.45) (width 0.2) (layer "F.Cu") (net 3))
 (segment (start 37.71 92.2) (end 35.571 90.061) (width 0.2) (layer "F.Cu") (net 3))
 (segment (start 32.601 71.7839) (end 32.601 59.05) (width 0.2) (layer "F.Cu") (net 3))
 (segment (start 114.25 49.45) (end 110.2 49.45) (width 0.2) (layer "F.Cu") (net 3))
 (segment (start 35.571 74.7539) (end 32.601 71.7839) (width 0.2) (layer "F.Cu") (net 3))
 (segment (start 77.14 56.4) (end 81.2 60.46) (width 0.2) (layer "F.Cu") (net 3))
 (via (at 89.25 49.3) (size 0.6) (drill 0.3) (layers "F.Cu" "B.Cu") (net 3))
 (segment (start 82.09 56.46) (end 82.09 60.46) (width 0.2) (layer "B.Cu") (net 3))
 (segment (start 81.2 61.35) (end 81.1 61.35) (width 0.2) (layer "B.Cu") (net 3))
 (segment (start 82.09 60.46) (end 81.2 61.35) (width 0.2) (layer "B.Cu") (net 3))
 (segment (start 89.25 49.3) (end 82.09 56.46) (width 0.2) (layer "B.Cu") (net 3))
 (segment (start 115.659 55.451) (end 97.92876 55.451) (width 0.2) (layer "F.Cu") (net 10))
 (segment (start 92.57776 50.1) (end 90.5 50.1) (width 0.2) (layer "F.Cu") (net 10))
 (segment (start 116.81 54.3) (end 115.659 55.451) (width 0.2) (layer "F.Cu") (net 10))
 (segment (start 97.92876 55.451) (end 92.57776 50.1) (width 0.2) (layer "F.Cu") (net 10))
 (via (at 90.5 50.1) (size 0.6) (drill 0.3) (layers "F.Cu" "B.Cu") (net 10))
 (segment (start 89.498943 48.699) (end 74.421 48.699) (width 0.2) (layer "B.Cu") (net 10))
 (segment (start 70.369 52.751) (end 69.379 52.751) (width 0.2) (layer "B.Cu") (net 10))
 (segment (start 74.421 48.699) (end 70.369 52.751) (width 0.2) (layer "B.Cu") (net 10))
 (segment (start 90.5 50.1) (end 90.5 49.700057) (width 0.2) (layer "B.Cu") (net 10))
 (segment (start 90.5 49.700057) (end 89.498943 48.699) (width 0.2) (layer "B.Cu") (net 10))
 (segment (start 69.379 52.751) (end 60.78 61.35) (width 0.2) (layer "B.Cu") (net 10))
 (segment (start 90.07 54.3) (end 38.55 54.3) (width 0.2) (layer "F.Cu") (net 19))
 (segment (start 38.55 54.3) (end 37.2 55.65) (width 0.2) (layer "F.Cu") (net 19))
 (via (at 37.2 55.65) (size 0.6) (drill 0.3) (layers "F.Cu" "B.Cu") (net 19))
 (segment (start 37.2 55.65) (end 36.37 56.48) (width 0.2) (layer "B.Cu") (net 19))
 (segment (start 36.37 56.48) (end 36.37 60.46) (width 0.2) (layer "B.Cu") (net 19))
 (segment (start 36.37 60.46) (end 35.48 61.35) (width 0.2) (layer "B.Cu") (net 19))
 (segment (start 35.48 61.35) (end 35.38 61.35) (width 0.2) (layer "B.Cu") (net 19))
 (segment (start 66.9 40.2) (end 66.9 36.22) (width 0.2) (layer "F.Cu") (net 20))
 (segment (start 92.61 54.3) (end 82.26 43.95) (width 0.2) (layer "F.Cu") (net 20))
 (segment (start 66.38 35.7) (end 65.88 35.7) (width 0.2) (layer "F.Cu") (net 20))
 (segment (start 70.65 43.95) (end 66.9 40.2) (width 0.2) (layer "F.Cu") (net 20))
 (segment (start 66.9 36.22) (end 66.38 35.7) (width 0.2) (layer "F.Cu") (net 20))
 (segment (start 82.26 43.95) (end 70.65 43.95) (width 0.2) (layer "F.Cu") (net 20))
 (segment (start 62 42.049955) (end 61.772538 41.822493) (width 0.2) (layer "B.Cu") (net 21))
 (segment (start 104.45 47.8) (end 67.75 47.8) (width 0.2) (layer "B.Cu") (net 21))
 (segment (start 61.772538 41.822493) (end 61.82 41.775031) (width 0.2) (layer "B.Cu") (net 21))
 (segment (start 61.82 41.775031) (end 61.82 36.22) (width 0.2) (layer "B.Cu") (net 21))
 (segment (start 118.2 88.45) (end 118.2 61.55) (width 0.2) (layer "B.Cu") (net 21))
 (segment (start 61.3 35.7) (end 60.8 35.7) (width 0.2) (layer "B.Cu") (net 21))
 (segment (start 67.75 47.8) (end 62 42.05) (width 0.2) (layer "B.Cu") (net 21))
 (segment (start 118.2 61.55) (end 104.45 47.8) (width 0.2) (layer "B.Cu") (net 21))
 (segment (start 62 42.05) (end 62 42.049955) (width 0.2) (layer "B.Cu") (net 21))
 (segment (start 121.95 92.2) (end 118.2 88.45) (width 0.2) (layer "B.Cu") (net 21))
 (segment (start 61.82 36.22) (end 61.3 35.7) (width 0.2) (layer "B.Cu") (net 21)))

